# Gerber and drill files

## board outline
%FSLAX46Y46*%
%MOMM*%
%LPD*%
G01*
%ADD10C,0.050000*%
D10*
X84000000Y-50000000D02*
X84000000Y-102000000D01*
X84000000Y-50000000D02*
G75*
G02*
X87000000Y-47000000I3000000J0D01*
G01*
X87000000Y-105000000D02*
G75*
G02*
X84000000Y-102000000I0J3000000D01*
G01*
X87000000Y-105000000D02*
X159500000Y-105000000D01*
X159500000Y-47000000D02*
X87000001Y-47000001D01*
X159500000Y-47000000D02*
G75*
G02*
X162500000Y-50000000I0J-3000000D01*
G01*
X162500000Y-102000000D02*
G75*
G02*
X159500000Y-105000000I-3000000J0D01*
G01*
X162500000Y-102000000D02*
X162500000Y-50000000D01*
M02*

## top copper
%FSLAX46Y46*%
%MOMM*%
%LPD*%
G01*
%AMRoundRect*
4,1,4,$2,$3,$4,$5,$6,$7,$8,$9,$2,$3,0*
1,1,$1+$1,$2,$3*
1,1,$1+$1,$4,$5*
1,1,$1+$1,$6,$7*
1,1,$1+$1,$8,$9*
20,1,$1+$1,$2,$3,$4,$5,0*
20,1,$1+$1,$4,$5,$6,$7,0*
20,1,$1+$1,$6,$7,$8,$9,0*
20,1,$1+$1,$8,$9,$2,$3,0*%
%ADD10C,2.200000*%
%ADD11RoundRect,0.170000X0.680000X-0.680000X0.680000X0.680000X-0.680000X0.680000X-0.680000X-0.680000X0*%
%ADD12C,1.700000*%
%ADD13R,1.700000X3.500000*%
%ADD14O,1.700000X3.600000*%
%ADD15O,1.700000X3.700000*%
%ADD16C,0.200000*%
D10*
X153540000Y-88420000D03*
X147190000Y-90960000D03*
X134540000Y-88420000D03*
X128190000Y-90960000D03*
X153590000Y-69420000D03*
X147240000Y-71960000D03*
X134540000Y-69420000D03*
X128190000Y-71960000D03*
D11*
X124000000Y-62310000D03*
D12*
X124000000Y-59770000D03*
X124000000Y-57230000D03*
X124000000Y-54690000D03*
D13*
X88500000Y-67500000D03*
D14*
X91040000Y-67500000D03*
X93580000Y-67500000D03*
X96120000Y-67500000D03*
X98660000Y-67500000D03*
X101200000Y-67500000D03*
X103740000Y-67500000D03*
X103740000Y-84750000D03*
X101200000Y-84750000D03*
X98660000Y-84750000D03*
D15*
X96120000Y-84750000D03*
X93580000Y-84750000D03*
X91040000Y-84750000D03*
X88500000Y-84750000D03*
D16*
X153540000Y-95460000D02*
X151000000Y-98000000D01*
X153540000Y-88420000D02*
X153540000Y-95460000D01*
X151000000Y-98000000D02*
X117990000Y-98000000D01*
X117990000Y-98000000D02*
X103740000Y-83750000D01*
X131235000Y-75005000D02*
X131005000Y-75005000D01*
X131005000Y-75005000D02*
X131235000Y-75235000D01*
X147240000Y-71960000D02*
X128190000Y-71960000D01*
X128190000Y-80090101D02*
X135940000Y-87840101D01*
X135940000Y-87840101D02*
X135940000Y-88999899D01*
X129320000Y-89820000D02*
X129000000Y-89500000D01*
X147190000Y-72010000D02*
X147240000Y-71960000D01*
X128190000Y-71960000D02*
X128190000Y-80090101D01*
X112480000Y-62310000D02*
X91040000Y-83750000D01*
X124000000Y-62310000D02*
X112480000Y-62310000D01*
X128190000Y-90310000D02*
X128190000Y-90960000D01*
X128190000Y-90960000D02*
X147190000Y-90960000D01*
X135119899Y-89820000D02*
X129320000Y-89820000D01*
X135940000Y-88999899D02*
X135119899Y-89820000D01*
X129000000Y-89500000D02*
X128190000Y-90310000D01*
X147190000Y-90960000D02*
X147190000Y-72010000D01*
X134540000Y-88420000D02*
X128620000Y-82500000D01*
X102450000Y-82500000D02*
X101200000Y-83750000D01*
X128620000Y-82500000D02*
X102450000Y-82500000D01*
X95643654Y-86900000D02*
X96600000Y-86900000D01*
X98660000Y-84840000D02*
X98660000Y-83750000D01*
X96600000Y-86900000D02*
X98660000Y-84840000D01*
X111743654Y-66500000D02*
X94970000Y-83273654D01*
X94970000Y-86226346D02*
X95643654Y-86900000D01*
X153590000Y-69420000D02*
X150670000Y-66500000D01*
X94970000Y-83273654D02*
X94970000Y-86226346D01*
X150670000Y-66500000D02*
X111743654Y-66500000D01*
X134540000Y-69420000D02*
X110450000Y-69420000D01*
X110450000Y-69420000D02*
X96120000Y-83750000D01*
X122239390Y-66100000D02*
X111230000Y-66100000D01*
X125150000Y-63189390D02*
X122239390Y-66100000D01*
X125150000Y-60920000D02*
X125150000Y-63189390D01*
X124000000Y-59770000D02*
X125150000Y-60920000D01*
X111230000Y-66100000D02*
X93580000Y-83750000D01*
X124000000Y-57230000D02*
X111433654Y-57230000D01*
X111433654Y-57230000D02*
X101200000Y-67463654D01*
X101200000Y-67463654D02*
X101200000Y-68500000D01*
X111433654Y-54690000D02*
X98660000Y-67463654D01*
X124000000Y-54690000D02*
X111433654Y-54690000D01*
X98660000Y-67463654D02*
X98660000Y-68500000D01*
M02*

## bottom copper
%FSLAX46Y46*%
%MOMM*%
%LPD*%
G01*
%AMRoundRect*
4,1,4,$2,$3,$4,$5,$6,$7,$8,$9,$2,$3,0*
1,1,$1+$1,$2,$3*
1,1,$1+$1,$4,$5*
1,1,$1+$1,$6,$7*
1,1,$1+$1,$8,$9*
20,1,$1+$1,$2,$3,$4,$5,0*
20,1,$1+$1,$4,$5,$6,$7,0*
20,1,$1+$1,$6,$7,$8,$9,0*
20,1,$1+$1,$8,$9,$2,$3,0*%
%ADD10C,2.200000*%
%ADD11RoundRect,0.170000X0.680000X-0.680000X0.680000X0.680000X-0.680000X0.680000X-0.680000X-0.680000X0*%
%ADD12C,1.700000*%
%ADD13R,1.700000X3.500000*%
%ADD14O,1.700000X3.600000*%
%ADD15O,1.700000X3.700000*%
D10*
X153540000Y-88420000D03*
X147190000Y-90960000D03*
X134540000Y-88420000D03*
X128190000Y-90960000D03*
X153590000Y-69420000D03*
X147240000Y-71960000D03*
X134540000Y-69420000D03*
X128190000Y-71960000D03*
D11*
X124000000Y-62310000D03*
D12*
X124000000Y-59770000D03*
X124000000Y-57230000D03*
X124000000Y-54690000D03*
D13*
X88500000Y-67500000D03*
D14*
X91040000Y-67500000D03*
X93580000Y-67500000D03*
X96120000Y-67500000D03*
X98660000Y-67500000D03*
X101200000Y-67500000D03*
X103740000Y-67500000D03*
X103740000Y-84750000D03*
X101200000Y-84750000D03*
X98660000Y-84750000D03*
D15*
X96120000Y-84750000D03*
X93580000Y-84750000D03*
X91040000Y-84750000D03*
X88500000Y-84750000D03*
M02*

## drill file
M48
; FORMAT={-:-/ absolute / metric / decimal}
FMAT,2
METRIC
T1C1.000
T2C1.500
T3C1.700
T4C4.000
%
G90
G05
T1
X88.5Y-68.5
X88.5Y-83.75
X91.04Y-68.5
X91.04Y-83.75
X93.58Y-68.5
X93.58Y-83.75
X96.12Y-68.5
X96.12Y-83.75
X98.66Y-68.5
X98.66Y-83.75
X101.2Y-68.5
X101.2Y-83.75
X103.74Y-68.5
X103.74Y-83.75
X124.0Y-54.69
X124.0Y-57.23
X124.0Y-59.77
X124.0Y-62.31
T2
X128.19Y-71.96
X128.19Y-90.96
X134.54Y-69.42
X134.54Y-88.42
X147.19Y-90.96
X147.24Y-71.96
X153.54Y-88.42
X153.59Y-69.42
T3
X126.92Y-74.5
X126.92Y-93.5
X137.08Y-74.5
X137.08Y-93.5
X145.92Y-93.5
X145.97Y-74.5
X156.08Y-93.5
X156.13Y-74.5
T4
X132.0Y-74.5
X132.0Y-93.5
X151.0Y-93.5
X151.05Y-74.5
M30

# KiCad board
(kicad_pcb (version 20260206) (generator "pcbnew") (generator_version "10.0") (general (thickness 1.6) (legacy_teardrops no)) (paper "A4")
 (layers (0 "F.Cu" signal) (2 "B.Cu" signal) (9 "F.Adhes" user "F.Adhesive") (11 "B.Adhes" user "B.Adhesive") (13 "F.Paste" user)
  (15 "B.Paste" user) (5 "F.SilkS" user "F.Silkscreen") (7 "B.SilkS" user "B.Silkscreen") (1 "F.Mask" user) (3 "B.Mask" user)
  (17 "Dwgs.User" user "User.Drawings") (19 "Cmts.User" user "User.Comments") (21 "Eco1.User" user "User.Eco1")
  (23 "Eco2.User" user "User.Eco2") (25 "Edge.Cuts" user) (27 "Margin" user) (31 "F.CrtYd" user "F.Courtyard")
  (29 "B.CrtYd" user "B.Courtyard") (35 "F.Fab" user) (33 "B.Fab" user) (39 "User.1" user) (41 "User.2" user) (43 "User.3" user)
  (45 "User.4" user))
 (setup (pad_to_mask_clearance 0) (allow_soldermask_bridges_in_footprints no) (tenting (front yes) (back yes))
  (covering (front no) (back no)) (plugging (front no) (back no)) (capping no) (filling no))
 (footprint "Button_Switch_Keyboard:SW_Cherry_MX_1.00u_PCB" (layer "F.Cu") (at 153.54 88.42)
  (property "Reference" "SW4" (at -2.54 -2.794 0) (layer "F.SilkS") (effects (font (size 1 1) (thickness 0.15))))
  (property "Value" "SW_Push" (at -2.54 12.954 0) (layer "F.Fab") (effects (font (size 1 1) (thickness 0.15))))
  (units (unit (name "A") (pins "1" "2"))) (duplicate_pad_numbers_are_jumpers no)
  (pad "" np_thru_hole circle (at -7.62 5.08) (size 1.7 1.7) (drill 1.7) (layers "*.Cu" "*.Mask"))
  (pad "" np_thru_hole circle (at -2.54 5.08) (size 4 4) (drill 4) (layers "*.Cu" "*.Mask"))
  (pad "" np_thru_hole circle (at 2.54 5.08) (size 1.7 1.7) (drill 1.7) (layers "*.Cu" "*.Mask"))
  (pad "1" thru_hole circle (at 0 0) (size 2.2 2.2) (drill 1.5) (layers "*.Cu" "*.Mask") (remove_unused_layers no)
   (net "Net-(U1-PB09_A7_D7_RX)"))
  (pad "2" thru_hole circle (at -6.35 2.54) (size 2.2 2.2) (drill 1.5) (layers "*.Cu" "*.Mask") (remove_unused_layers no) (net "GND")))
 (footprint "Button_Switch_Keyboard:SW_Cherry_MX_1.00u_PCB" (layer "F.Cu") (at 134.54 88.42)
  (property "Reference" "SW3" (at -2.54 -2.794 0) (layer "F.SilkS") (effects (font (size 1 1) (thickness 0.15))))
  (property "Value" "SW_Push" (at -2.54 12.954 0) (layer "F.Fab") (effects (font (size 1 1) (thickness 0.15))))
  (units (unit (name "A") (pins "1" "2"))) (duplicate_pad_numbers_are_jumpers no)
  (pad "" np_thru_hole circle (at -7.62 5.08) (size 1.7 1.7) (drill 1.7) (layers "*.Cu" "*.Mask"))
  (pad "" np_thru_hole circle (at -2.54 5.08) (size 4 4) (drill 4) (layers "*.Cu" "*.Mask"))
  (pad "" np_thru_hole circle (at 2.54 5.08) (size 1.7 1.7) (drill 1.7) (layers "*.Cu" "*.Mask"))
  (pad "1" thru_hole circle (at 0 0) (size 2.2 2.2) (drill 1.5) (layers "*.Cu" "*.Mask") (remove_unused_layers no)
   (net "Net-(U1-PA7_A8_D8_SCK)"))
  (pad "2" thru_hole circle (at -6.35 2.54) (size 2.2 2.2) (drill 1.5) (layers "*.Cu" "*.Mask") (remove_unused_layers no) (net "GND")))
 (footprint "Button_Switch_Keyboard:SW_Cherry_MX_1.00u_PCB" (layer "F.Cu") (at 153.59 69.42)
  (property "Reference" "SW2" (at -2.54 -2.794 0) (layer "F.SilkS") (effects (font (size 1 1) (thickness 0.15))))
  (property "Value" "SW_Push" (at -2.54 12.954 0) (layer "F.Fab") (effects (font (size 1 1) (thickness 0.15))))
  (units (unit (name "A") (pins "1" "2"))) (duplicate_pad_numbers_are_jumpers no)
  (pad "" np_thru_hole circle (at -7.62 5.08) (size 1.7 1.7) (drill 1.7) (layers "*.Cu" "*.Mask"))
  (pad "" np_thru_hole circle (at -2.54 5.08) (size 4 4) (drill 4) (layers "*.Cu" "*.Mask"))
  (pad "" np_thru_hole circle (at 2.54 5.08) (size 1.7 1.7) (drill 1.7) (layers "*.Cu" "*.Mask"))
  (pad "1" thru_hole circle (at 0 0) (size 2.2 2.2) (drill 1.5) (layers "*.Cu" "*.Mask") (remove_unused_layers no)
   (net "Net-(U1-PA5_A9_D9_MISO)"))
  (pad "2" thru_hole circle (at -6.35 2.54) (size 2.2 2.2) (drill 1.5) (layers "*.Cu" "*.Mask") (remove_unused_layers no) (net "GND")))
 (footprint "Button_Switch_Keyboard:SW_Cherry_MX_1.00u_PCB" (layer "F.Cu") (at 134.54 69.42)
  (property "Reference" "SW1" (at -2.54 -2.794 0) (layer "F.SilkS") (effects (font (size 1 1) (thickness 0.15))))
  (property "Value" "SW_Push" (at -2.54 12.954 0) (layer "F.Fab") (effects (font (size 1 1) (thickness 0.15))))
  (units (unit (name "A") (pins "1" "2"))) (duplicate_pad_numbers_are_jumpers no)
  (pad "" np_thru_hole circle (at -7.62 5.08) (size 1.7 1.7) (drill 1.7) (layers "*.Cu" "*.Mask"))
  (pad "" np_thru_hole circle (at -2.54 5.08) (size 4 4) (drill 4) (layers "*.Cu" "*.Mask"))
  (pad "" np_thru_hole circle (at 2.54 5.08) (size 1.7 1.7) (drill 1.7) (layers "*.Cu" "*.Mask"))
  (pad "1" thru_hole circle (at 0 0) (size 2.2 2.2) (drill 1.5) (layers "*.Cu" "*.Mask") (remove_unused_layers no)
   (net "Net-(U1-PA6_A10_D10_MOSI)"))
  (pad "2" thru_hole circle (at -6.35 2.54) (size 2.2 2.2) (drill 1.5) (layers "*.Cu" "*.Mask") (remove_unused_layers no) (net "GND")))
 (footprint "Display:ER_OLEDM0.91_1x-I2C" (layer "F.Cu") (at 124 62.31 90)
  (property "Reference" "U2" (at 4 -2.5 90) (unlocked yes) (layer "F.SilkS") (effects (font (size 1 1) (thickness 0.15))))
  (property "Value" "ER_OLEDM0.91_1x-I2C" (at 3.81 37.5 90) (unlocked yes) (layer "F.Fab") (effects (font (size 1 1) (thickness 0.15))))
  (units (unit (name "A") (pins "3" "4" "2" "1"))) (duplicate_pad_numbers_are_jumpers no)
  (pad "1" thru_hole roundrect (at 0 0 90) (size 1.7 1.7) (drill 1) (layers "*.Cu" "*.Mask") (remove_unused_layers no)
   (roundrect_rratio 0.1) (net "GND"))
  (pad "2" thru_hole circle (at 2.54 0 90) (size 1.7 1.7) (drill 1) (layers "*.Cu" "*.Mask") (remove_unused_layers no) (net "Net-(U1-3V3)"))
  (pad "3" thru_hole circle (at 5.08 0 90) (size 1.7 1.7) (drill 1) (layers "*.Cu" "*.Mask") (remove_unused_layers no)
   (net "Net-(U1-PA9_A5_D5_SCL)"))
  (pad "4" thru_hole circle (at 7.62 0 90) (size 1.7 1.7) (drill 1) (layers "*.Cu" "*.Mask") (remove_unused_layers no)
   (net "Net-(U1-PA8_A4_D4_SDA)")))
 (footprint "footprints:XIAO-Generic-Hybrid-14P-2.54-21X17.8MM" (layer "B.Cu") (at 96.12 76.125 -90)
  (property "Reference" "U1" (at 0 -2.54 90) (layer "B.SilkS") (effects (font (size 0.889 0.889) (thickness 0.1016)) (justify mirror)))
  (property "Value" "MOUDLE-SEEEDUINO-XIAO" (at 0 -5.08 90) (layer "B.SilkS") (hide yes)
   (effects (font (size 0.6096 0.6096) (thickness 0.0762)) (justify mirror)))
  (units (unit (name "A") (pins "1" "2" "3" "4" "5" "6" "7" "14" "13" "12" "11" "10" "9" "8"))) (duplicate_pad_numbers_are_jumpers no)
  (pad "1" thru_hole rect (at -7.625 7.62 270) (size 3.5 1.7) (drill 1 (offset -1 0)) (layers "*.Cu" "*.Mask") (remove_unused_layers no)
   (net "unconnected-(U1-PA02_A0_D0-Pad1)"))
  (pad "2" thru_hole oval (at -7.625 5.08 270) (size 3.6 1.7) (drill 1 (offset -1 0)) (layers "*.Cu" "*.Mask") (remove_unused_layers no)
   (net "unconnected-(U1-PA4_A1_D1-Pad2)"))
  (pad "3" thru_hole oval (at -7.625 2.54 270) (size 3.6 1.7) (drill 1 (offset -1 0)) (layers "*.Cu" "*.Mask") (remove_unused_layers no)
   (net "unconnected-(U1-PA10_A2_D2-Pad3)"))
  (pad "4" thru_hole oval (at -7.625 0 270) (size 3.6 1.7) (drill 1 (offset -1 0)) (layers "*.Cu" "*.Mask") (remove_unused_layers no)
   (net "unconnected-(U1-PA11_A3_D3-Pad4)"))
  (pad "5" thru_hole oval (at -7.625 -2.54 270) (size 3.6 1.7) (drill 1 (offset -1 0)) (layers "*.Cu" "*.Mask") (remove_unused_layers no)
   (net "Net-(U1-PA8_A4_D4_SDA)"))
  (pad "6" thru_hole oval (at -7.625 -5.08 90) (size 3.6 1.7) (drill 1 (offset 1 0)) (layers "*.Cu" "*.Mask") (remove_unused_layers no)
   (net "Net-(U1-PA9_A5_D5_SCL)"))
  (pad "7" thru_hole oval (at -7.625 -7.62 270) (size 3.6 1.7) (drill 1 (offset -1 0)) (layers "*.Cu" "*.Mask") (remove_unused_layers no)
   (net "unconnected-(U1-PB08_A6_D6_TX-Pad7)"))
  (pad "8" thru_hole oval (at 7.625 -7.62 270) (size 3.6 1.7) (drill 1 (offset 1 0)) (layers "*.Cu" "*.Mask") (remove_unused_layers no)
   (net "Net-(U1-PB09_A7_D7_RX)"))
  (pad "9" thru_hole oval (at 7.625 -5.08 270) (size 3.6 1.7) (drill 1 (offset 1 0)) (layers "*.Cu" "*.Mask") (remove_unused_layers no)
   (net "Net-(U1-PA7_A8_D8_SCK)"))
  (pad "10" thru_hole oval (at 7.625 -2.54 270) (size 3.6 1.7) (drill 1 (offset 1 0)) (layers "*.Cu" "*.Mask") (remove_unused_layers no)
   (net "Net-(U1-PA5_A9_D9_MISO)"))
  (pad "11" thru_hole oval (at 7.625 0 270) (size 3.7 1.7) (drill 1 (offset 1 0)) (layers "*.Cu" "*.Mask") (remove_unused_layers no)
   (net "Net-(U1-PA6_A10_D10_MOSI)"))
  (pad "12" thru_hole oval (at 7.625 2.54 270) (size 3.7 1.7) (drill 1 (offset 1 0)) (layers "*.Cu" "*.Mask") (remove_unused_layers no)
   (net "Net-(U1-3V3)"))
  (pad "13" thru_hole oval (at 7.625 5.08 270) (size 3.7 1.7) (drill 1 (offset 1 0)) (layers "*.Cu" "*.Mask") (remove_unused_layers no)
   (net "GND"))
  (pad "14" thru_hole oval (at 7.625 7.62 270) (size 3.7 1.7) (drill 1 (offset 1 0)) (layers "*.Cu" "*.Mask") (remove_unused_layers no)
   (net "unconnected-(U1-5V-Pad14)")))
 (gr_line (start 84 50) (end 84 102) (stroke (width 0.05) (type default)) (layer "Edge.Cuts"))
 (gr_arc (start 84 50) (mid 84.87868 47.87868) (end 87 47) (stroke (width 0.05) (type default)) (layer "Edge.Cuts"))
 (gr_arc (start 87 105) (mid 84.87868 104.12132) (end 84 102) (stroke (width 0.05) (type default)) (layer "Edge.Cuts"))
 (gr_line (start 87 105) (end 159.5 105) (stroke (width 0.05) (type default)) (layer "Edge.Cuts"))
 (gr_line (start 159.5 47) (end 87.000001 47.000001) (stroke (width 0.05) (type default)) (layer "Edge.Cuts"))
 (gr_arc (start 159.5 47) (mid 161.62132 47.87868) (end 162.5 50) (stroke (width 0.05) (type default)) (layer "Edge.Cuts"))
 (gr_arc (start 162.5 102) (mid 161.62132 104.12132) (end 159.5 105) (stroke (width 0.05) (type default)) (layer "Edge.Cuts"))
 (gr_line (start 162.5 102) (end 162.5 50) (stroke (width 0.05) (type default)) (layer "Edge.Cuts"))
 (segment (start 153.54 95.46) (end 151 98) (width 0.2) (layer "F.Cu") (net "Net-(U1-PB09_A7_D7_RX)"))
 (segment (start 153.54 88.42) (end 153.54 95.46) (width 0.2) (layer "F.Cu") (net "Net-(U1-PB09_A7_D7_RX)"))
 (segment (start 151 98) (end 117.99 98) (width 0.2) (layer "F.Cu") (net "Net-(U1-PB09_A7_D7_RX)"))
 (segment (start 117.99 98) (end 103.74 83.75) (width 0.2) (layer "F.Cu") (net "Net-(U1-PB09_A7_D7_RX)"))
 (segment (start 131.235 75.005) (end 131.005 75.005) (width 0.2) (layer "F.Cu") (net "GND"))
 (segment (start 131.005 75.005) (end 131.235 75.235) (width 0.2) (layer "F.Cu") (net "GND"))
 (segment (start 147.24 71.96) (end 128.19 71.96) (width 0.2) (layer "F.Cu") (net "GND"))
 (segment (start 128.19 80.090101) (end 135.94 87.840101) (width 0.2) (layer "F.Cu") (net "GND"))
 (segment (start 135.94 87.840101) (end 135.94 88.999899) (width 0.2) (layer "F.Cu") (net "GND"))
 (segment (start 129.32 89.82) (end 129 89.5) (width 0.2) (layer "F.Cu") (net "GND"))
 (segment (start 147.19 72.01) (end 147.24 71.96) (width 0.2) (layer "F.Cu") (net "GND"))
 (segment (start 128.19 71.96) (end 128.19 80.090101) (width 0.2) (layer "F.Cu") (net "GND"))
 (segment (start 112.48 62.31) (end 91.04 83.75) (width 0.2) (layer "F.Cu") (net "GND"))
 (segment (start 124 62.31) (end 112.48 62.31) (width 0.2) (layer "F.Cu") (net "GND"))
 (segment (start 128.19 90.31) (end 128.19 90.96) (width 0.2) (layer "F.Cu") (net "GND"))
 (segment (start 128.19 90.96) (end 147.19 90.96) (width 0.2) (layer "F.Cu") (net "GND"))
 (segment (start 135.119899 89.82) (end 129.32 89.82) (width 0.2) (layer "F.Cu") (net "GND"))
 (segment (start 135.94 88.999899) (end 135.119899 89.82) (width 0.2) (layer "F.Cu") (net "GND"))
 (segment (start 129 89.5) (end 128.19 90.31) (width 0.2) (layer "F.Cu") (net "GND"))
 (segment (start 147.19 90.96) (end 147.19 72.01) (width 0.2) (layer "F.Cu") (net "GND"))
 (segment (start 134.54 88.42) (end 128.62 82.5) (width 0.2) (layer "F.Cu") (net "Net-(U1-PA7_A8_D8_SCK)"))
 (segment (start 102.45 82.5) (end 101.2 83.75) (width 0.2) (layer "F.Cu") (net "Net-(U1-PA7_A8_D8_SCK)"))
 (segment (start 128.62 82.5) (end 102.45 82.5) (width 0.2) (layer "F.Cu") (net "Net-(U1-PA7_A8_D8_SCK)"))
 (segment (start 95.643654 86.9) (end 96.6 86.9) (width 0.2) (layer "F.Cu") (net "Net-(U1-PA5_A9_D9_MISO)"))
 (segment (start 98.66 84.84) (end 98.66 83.75) (width 0.2) (layer "F.Cu") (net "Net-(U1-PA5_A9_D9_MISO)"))
 (segment (start 96.6 86.9) (end 98.66 84.84) (width 0.2) (layer "F.Cu") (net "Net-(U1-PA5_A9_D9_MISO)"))
 (segment (start 111.743654 66.5) (end 94.97 83.273654) (width 0.2) (layer "F.Cu") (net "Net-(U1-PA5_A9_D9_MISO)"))
 (segment (start 94.97 86.226346) (end 95.643654 86.9) (width 0.2) (layer "F.Cu") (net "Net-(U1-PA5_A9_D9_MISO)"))
 (segment (start 153.59 69.42) (end 150.67 66.5) (width 0.2) (layer "F.Cu") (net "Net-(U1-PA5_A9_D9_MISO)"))
 (segment (start 94.97 83.273654) (end 94.97 86.226346) (width 0.2) (layer "F.Cu") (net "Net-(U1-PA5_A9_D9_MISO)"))
 (segment (start 150.67 66.5) (end 111.743654 66.5) (width 0.2) (layer "F.Cu") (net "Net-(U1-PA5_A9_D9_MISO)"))
 (segment (start 134.54 69.42) (end 110.45 69.42) (width 0.2) (layer "F.Cu") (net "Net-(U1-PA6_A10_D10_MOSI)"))
 (segment (start 110.45 69.42) (end 96.12 83.75) (width 0.2) (layer "F.Cu") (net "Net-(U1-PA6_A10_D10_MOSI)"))
 (segment (start 122.23939 66.1) (end 111.23 66.1) (width 0.2) (layer "F.Cu") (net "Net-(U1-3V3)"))
 (segment (start 125.15 63.18939) (end 122.23939 66.1) (width 0.2) (layer "F.Cu") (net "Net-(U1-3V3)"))
 (segment (start 125.15 60.92) (end 125.15 63.18939) (width 0.2) (layer "F.Cu") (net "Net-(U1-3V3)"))
 (segment (start 124 59.77) (end 125.15 60.92) (width 0.2) (layer "F.Cu") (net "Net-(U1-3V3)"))
 (segment (start 111.23 66.1) (end 93.58 83.75) (width 0.2) (layer "F.Cu") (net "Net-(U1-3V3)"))
 (segment (start 124 57.23) (end 111.433654 57.23) (width 0.2) (layer "F.Cu") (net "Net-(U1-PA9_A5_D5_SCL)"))
 (segment (start 111.433654 57.23) (end 101.2 67.463654) (width 0.2) (layer "F.Cu") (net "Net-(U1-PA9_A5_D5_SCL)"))
 (segment (start 101.2 67.463654) (end 101.2 68.5) (width 0.2) (layer "F.Cu") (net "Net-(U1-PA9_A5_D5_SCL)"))
 (segment (start 111.433654 54.69) (end 98.66 67.463654) (width 0.2) (layer "F.Cu") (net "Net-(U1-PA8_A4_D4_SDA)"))
 (segment (start 124 54.69) (end 111.433654 54.69) (width 0.2) (layer "F.Cu") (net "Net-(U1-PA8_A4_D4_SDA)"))
 (segment (start 98.66 67.463654) (end 98.66 68.5) (width 0.2) (layer "F.Cu") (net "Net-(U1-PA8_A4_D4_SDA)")))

